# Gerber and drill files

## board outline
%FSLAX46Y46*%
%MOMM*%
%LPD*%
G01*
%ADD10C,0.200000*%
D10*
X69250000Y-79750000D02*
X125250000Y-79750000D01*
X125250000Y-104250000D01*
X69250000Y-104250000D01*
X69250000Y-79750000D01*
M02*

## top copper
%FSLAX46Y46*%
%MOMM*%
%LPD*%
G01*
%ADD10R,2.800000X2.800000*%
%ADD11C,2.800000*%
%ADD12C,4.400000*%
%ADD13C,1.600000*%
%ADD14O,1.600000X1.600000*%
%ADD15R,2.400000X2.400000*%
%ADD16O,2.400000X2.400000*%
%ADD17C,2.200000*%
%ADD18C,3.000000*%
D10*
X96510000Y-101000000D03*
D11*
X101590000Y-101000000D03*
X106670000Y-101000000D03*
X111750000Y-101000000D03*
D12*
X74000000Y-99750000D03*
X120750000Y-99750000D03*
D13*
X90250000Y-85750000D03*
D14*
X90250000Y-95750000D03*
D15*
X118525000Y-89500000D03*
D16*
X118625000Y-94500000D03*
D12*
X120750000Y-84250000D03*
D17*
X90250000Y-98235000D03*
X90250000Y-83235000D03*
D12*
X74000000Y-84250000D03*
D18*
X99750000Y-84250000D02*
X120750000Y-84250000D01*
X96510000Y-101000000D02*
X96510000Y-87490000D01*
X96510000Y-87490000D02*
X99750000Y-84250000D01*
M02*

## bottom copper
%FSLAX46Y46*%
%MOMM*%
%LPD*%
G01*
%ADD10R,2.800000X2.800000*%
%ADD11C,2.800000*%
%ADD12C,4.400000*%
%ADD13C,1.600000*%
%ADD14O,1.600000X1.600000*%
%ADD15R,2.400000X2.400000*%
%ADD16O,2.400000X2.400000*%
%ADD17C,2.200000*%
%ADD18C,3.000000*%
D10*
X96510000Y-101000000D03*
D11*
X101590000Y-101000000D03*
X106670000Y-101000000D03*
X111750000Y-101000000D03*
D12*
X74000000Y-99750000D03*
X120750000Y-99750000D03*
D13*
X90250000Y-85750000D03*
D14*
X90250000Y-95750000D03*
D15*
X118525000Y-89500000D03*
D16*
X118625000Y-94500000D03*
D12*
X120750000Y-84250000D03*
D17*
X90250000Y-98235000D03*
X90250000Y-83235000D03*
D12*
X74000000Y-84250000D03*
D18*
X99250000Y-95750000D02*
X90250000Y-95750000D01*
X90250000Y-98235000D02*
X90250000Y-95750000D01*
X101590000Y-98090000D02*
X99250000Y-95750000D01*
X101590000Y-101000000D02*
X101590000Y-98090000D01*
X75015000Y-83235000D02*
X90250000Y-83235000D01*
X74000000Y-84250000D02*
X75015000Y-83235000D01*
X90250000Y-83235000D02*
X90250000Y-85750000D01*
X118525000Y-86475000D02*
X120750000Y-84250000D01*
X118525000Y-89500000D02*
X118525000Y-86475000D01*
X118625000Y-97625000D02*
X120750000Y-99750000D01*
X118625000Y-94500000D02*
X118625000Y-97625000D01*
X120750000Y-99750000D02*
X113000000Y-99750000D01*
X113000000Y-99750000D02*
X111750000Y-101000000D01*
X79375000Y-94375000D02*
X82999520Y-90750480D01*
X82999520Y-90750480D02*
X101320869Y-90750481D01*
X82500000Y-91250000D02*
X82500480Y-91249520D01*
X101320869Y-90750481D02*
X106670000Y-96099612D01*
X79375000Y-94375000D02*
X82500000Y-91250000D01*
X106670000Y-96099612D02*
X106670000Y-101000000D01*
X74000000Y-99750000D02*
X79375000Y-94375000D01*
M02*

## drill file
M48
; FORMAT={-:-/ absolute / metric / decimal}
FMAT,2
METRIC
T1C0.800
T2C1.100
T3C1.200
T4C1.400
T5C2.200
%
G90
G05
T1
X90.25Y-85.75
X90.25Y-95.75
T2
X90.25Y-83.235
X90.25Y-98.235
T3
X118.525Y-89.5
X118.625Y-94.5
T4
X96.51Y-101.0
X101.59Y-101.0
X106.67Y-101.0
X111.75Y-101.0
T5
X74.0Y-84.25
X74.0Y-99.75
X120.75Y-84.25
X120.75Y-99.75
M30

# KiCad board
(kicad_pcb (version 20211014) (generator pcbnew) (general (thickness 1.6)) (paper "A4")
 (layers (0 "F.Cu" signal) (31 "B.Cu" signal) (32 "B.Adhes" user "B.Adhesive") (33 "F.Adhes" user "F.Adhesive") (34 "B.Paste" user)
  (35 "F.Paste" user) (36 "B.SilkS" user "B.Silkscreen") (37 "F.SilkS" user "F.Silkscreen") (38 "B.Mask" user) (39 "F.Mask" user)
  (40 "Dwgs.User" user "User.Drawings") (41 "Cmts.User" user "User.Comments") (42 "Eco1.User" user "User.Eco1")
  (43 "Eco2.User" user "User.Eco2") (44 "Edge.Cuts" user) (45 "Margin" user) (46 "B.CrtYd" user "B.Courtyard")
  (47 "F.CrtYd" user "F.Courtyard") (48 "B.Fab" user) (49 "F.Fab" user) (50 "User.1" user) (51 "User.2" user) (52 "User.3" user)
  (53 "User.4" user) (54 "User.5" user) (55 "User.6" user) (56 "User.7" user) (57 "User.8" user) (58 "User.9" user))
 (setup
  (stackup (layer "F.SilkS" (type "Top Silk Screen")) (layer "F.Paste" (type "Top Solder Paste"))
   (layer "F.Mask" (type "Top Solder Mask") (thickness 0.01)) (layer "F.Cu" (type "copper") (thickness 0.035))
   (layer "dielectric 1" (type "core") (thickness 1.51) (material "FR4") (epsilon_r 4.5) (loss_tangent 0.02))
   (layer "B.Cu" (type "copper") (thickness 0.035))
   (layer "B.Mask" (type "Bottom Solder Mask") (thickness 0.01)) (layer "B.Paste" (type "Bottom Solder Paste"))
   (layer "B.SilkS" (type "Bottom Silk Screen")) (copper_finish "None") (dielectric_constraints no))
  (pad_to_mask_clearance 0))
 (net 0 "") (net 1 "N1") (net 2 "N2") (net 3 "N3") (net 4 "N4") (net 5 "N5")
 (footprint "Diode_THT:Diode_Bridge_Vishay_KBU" (layer "F.Cu") (at 111.75 101 180)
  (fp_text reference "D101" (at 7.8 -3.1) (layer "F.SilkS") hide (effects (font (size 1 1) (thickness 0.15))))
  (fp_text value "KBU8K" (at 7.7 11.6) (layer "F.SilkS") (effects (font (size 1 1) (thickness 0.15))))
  (pad "1" thru_hole rect (at 15.24 0 180) (size 2.8 2.8) (drill 1.4) (layers *.Cu *.Mask) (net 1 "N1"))
  (pad "2" thru_hole circle (at 10.16 0 180) (size 2.8 2.8) (drill 1.4) (layers *.Cu *.Mask) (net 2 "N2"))
  (pad "3" thru_hole circle (at 5.08 0 180) (size 2.8 2.8) (drill 1.4) (layers *.Cu *.Mask) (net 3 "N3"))
  (pad "4" thru_hole circle (at 0 0 180) (size 2.8 2.8) (drill 1.4) (layers *.Cu *.Mask) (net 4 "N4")))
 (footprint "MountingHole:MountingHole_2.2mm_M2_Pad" (layer "F.Cu") (at 74 99.75)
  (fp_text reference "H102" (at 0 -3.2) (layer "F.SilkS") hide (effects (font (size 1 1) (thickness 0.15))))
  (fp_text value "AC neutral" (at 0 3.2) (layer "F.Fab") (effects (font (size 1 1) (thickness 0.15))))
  (pad "1" thru_hole circle (at 0 0) (size 4.4 4.4) (drill 2.2) (layers *.Cu *.Mask) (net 3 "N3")))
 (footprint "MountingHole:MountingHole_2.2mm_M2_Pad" (layer "F.Cu") (at 120.75 99.75 180)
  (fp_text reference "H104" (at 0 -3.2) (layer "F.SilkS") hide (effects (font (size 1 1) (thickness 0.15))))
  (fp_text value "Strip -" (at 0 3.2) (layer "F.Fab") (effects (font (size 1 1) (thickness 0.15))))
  (pad "1" thru_hole circle (at 0 0 180) (size 4.4 4.4) (drill 2.2) (layers *.Cu *.Mask) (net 4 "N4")))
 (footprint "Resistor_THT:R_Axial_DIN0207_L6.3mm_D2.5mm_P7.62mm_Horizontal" (layer "F.Cu") (at 90.25 86.95 -90)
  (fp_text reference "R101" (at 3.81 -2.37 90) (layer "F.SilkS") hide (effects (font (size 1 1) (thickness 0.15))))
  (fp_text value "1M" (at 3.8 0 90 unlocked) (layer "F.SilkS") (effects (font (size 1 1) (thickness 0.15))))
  (pad "1" thru_hole circle (at -1.2 0 270) (size 1.6 1.6) (drill 0.8) (layers *.Cu *.Mask) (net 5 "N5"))
  (pad "2" thru_hole oval (at 8.8 0 270) (size 1.6 1.6) (drill 0.8) (layers *.Cu *.Mask) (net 2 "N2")))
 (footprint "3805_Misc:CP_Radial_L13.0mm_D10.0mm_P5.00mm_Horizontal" (layer "F.Cu") (at 118.525 92)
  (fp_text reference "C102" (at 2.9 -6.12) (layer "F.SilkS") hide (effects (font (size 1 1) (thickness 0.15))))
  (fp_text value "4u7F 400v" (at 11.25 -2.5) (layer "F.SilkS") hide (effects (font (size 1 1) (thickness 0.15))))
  (pad "1" thru_hole rect (at 0 -2.5) (size 2.4 2.4) (drill 1.2) (layers *.Cu *.Mask) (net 1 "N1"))
  (pad "2" thru_hole oval (at 0.1 2.5) (size 2.4 2.4) (drill 1.2) (layers *.Cu *.Mask) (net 4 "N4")))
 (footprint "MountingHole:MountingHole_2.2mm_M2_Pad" (layer "F.Cu") (at 120.75 84.25)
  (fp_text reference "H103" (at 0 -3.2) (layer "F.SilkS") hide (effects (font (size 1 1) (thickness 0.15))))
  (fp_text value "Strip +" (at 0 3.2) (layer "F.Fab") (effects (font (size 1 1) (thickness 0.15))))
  (pad "1" thru_hole circle (at 0 0) (size 4.4 4.4) (drill 2.2) (layers *.Cu *.Mask) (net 1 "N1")))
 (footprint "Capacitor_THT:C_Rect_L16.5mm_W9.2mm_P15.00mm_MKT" (layer "F.Cu") (at 90.25 98.235 90)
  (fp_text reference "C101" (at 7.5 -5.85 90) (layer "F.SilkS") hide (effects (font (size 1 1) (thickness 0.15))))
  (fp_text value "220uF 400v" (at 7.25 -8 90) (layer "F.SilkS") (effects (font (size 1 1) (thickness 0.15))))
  (pad "1" thru_hole circle (at 0 0 90) (size 2.2 2.2) (drill 1.1) (layers *.Cu *.Mask) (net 2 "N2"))
  (pad "2" thru_hole circle (at 15 0 90) (size 2.2 2.2) (drill 1.1) (layers *.Cu *.Mask) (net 5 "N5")))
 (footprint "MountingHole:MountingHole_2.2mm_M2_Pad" (layer "F.Cu") (at 74 84.25)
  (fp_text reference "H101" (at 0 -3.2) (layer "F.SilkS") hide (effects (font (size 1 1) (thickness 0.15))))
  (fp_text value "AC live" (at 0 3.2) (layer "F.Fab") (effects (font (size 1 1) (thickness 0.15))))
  (pad "1" thru_hole circle (at 0 0) (size 4.4 4.4) (drill 2.2) (layers *.Cu *.Mask) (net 5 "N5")))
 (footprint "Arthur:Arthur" (layer "B.Cu") (at 83.5 99 180)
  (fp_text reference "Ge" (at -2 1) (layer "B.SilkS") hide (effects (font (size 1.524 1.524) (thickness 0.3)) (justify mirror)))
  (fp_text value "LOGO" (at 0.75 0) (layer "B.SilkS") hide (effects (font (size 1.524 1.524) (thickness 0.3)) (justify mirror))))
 (gr_rect (start 69.25 79.75) (end 125.25 104.25) (layer "Edge.Cuts") (width 0.2) (fill none))
 (segment (start 99.25 95.75) (end 90.25 95.75) (width 3) (layer "B.Cu") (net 2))
 (segment (start 90.25 98.235) (end 90.25 95.75) (width 3) (layer "B.Cu") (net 2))
 (segment (start 101.59 98.09) (end 99.25 95.75) (width 3) (layer "B.Cu") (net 2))
 (segment (start 101.59 101) (end 101.59 98.09) (width 3) (layer "B.Cu") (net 2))
 (segment (start 75.015 83.235) (end 90.25 83.235) (width 3) (layer "B.Cu") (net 5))
 (segment (start 74 84.25) (end 75.015 83.235) (width 3) (layer "B.Cu") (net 5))
 (segment (start 90.25 83.235) (end 90.25 85.75) (width 3) (layer "B.Cu") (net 5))
 (segment (start 99.75 84.25) (end 120.75 84.25) (width 3) (layer "F.Cu") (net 1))
 (segment (start 96.51 101) (end 96.51 87.49) (width 3) (layer "F.Cu") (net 1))
 (segment (start 96.51 87.49) (end 99.75 84.25) (width 3) (layer "F.Cu") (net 1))
 (segment (start 118.525 86.475) (end 120.75 84.25) (width 3) (layer "B.Cu") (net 1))
 (segment (start 118.525 89.5) (end 118.525 86.475) (width 3) (layer "B.Cu") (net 1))
 (segment (start 118.625 97.625) (end 120.75 99.75) (width 3) (layer "B.Cu") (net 4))
 (segment (start 118.625 94.5) (end 118.625 97.625) (width 3) (layer "B.Cu") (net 4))
 (segment (start 120.75 99.75) (end 113 99.75) (width 3) (layer "B.Cu") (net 4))
 (segment (start 113 99.75) (end 111.75 101) (width 3) (layer "B.Cu") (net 4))
 (segment (start 79.375 94.375) (end 82.99952 90.75048) (width 3) (layer "B.Cu") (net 3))
 (segment (start 82.99952 90.75048) (end 101.320869 90.750481) (width 3) (layer "B.Cu") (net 3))
 (segment (start 82.5 91.25) (end 82.50048 91.24952) (width 3) (layer "B.Cu") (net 3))
 (segment (start 101.320869 90.750481) (end 106.67 96.099612) (width 3) (layer "B.Cu") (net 3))
 (segment (start 79.375 94.375) (end 82.5 91.25) (width 3) (layer "B.Cu") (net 3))
 (segment (start 106.67 96.099612) (end 106.67 101) (width 3) (layer "B.Cu") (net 3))
 (segment (start 74 99.75) (end 79.375 94.375) (width 3) (layer "B.Cu") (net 3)))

